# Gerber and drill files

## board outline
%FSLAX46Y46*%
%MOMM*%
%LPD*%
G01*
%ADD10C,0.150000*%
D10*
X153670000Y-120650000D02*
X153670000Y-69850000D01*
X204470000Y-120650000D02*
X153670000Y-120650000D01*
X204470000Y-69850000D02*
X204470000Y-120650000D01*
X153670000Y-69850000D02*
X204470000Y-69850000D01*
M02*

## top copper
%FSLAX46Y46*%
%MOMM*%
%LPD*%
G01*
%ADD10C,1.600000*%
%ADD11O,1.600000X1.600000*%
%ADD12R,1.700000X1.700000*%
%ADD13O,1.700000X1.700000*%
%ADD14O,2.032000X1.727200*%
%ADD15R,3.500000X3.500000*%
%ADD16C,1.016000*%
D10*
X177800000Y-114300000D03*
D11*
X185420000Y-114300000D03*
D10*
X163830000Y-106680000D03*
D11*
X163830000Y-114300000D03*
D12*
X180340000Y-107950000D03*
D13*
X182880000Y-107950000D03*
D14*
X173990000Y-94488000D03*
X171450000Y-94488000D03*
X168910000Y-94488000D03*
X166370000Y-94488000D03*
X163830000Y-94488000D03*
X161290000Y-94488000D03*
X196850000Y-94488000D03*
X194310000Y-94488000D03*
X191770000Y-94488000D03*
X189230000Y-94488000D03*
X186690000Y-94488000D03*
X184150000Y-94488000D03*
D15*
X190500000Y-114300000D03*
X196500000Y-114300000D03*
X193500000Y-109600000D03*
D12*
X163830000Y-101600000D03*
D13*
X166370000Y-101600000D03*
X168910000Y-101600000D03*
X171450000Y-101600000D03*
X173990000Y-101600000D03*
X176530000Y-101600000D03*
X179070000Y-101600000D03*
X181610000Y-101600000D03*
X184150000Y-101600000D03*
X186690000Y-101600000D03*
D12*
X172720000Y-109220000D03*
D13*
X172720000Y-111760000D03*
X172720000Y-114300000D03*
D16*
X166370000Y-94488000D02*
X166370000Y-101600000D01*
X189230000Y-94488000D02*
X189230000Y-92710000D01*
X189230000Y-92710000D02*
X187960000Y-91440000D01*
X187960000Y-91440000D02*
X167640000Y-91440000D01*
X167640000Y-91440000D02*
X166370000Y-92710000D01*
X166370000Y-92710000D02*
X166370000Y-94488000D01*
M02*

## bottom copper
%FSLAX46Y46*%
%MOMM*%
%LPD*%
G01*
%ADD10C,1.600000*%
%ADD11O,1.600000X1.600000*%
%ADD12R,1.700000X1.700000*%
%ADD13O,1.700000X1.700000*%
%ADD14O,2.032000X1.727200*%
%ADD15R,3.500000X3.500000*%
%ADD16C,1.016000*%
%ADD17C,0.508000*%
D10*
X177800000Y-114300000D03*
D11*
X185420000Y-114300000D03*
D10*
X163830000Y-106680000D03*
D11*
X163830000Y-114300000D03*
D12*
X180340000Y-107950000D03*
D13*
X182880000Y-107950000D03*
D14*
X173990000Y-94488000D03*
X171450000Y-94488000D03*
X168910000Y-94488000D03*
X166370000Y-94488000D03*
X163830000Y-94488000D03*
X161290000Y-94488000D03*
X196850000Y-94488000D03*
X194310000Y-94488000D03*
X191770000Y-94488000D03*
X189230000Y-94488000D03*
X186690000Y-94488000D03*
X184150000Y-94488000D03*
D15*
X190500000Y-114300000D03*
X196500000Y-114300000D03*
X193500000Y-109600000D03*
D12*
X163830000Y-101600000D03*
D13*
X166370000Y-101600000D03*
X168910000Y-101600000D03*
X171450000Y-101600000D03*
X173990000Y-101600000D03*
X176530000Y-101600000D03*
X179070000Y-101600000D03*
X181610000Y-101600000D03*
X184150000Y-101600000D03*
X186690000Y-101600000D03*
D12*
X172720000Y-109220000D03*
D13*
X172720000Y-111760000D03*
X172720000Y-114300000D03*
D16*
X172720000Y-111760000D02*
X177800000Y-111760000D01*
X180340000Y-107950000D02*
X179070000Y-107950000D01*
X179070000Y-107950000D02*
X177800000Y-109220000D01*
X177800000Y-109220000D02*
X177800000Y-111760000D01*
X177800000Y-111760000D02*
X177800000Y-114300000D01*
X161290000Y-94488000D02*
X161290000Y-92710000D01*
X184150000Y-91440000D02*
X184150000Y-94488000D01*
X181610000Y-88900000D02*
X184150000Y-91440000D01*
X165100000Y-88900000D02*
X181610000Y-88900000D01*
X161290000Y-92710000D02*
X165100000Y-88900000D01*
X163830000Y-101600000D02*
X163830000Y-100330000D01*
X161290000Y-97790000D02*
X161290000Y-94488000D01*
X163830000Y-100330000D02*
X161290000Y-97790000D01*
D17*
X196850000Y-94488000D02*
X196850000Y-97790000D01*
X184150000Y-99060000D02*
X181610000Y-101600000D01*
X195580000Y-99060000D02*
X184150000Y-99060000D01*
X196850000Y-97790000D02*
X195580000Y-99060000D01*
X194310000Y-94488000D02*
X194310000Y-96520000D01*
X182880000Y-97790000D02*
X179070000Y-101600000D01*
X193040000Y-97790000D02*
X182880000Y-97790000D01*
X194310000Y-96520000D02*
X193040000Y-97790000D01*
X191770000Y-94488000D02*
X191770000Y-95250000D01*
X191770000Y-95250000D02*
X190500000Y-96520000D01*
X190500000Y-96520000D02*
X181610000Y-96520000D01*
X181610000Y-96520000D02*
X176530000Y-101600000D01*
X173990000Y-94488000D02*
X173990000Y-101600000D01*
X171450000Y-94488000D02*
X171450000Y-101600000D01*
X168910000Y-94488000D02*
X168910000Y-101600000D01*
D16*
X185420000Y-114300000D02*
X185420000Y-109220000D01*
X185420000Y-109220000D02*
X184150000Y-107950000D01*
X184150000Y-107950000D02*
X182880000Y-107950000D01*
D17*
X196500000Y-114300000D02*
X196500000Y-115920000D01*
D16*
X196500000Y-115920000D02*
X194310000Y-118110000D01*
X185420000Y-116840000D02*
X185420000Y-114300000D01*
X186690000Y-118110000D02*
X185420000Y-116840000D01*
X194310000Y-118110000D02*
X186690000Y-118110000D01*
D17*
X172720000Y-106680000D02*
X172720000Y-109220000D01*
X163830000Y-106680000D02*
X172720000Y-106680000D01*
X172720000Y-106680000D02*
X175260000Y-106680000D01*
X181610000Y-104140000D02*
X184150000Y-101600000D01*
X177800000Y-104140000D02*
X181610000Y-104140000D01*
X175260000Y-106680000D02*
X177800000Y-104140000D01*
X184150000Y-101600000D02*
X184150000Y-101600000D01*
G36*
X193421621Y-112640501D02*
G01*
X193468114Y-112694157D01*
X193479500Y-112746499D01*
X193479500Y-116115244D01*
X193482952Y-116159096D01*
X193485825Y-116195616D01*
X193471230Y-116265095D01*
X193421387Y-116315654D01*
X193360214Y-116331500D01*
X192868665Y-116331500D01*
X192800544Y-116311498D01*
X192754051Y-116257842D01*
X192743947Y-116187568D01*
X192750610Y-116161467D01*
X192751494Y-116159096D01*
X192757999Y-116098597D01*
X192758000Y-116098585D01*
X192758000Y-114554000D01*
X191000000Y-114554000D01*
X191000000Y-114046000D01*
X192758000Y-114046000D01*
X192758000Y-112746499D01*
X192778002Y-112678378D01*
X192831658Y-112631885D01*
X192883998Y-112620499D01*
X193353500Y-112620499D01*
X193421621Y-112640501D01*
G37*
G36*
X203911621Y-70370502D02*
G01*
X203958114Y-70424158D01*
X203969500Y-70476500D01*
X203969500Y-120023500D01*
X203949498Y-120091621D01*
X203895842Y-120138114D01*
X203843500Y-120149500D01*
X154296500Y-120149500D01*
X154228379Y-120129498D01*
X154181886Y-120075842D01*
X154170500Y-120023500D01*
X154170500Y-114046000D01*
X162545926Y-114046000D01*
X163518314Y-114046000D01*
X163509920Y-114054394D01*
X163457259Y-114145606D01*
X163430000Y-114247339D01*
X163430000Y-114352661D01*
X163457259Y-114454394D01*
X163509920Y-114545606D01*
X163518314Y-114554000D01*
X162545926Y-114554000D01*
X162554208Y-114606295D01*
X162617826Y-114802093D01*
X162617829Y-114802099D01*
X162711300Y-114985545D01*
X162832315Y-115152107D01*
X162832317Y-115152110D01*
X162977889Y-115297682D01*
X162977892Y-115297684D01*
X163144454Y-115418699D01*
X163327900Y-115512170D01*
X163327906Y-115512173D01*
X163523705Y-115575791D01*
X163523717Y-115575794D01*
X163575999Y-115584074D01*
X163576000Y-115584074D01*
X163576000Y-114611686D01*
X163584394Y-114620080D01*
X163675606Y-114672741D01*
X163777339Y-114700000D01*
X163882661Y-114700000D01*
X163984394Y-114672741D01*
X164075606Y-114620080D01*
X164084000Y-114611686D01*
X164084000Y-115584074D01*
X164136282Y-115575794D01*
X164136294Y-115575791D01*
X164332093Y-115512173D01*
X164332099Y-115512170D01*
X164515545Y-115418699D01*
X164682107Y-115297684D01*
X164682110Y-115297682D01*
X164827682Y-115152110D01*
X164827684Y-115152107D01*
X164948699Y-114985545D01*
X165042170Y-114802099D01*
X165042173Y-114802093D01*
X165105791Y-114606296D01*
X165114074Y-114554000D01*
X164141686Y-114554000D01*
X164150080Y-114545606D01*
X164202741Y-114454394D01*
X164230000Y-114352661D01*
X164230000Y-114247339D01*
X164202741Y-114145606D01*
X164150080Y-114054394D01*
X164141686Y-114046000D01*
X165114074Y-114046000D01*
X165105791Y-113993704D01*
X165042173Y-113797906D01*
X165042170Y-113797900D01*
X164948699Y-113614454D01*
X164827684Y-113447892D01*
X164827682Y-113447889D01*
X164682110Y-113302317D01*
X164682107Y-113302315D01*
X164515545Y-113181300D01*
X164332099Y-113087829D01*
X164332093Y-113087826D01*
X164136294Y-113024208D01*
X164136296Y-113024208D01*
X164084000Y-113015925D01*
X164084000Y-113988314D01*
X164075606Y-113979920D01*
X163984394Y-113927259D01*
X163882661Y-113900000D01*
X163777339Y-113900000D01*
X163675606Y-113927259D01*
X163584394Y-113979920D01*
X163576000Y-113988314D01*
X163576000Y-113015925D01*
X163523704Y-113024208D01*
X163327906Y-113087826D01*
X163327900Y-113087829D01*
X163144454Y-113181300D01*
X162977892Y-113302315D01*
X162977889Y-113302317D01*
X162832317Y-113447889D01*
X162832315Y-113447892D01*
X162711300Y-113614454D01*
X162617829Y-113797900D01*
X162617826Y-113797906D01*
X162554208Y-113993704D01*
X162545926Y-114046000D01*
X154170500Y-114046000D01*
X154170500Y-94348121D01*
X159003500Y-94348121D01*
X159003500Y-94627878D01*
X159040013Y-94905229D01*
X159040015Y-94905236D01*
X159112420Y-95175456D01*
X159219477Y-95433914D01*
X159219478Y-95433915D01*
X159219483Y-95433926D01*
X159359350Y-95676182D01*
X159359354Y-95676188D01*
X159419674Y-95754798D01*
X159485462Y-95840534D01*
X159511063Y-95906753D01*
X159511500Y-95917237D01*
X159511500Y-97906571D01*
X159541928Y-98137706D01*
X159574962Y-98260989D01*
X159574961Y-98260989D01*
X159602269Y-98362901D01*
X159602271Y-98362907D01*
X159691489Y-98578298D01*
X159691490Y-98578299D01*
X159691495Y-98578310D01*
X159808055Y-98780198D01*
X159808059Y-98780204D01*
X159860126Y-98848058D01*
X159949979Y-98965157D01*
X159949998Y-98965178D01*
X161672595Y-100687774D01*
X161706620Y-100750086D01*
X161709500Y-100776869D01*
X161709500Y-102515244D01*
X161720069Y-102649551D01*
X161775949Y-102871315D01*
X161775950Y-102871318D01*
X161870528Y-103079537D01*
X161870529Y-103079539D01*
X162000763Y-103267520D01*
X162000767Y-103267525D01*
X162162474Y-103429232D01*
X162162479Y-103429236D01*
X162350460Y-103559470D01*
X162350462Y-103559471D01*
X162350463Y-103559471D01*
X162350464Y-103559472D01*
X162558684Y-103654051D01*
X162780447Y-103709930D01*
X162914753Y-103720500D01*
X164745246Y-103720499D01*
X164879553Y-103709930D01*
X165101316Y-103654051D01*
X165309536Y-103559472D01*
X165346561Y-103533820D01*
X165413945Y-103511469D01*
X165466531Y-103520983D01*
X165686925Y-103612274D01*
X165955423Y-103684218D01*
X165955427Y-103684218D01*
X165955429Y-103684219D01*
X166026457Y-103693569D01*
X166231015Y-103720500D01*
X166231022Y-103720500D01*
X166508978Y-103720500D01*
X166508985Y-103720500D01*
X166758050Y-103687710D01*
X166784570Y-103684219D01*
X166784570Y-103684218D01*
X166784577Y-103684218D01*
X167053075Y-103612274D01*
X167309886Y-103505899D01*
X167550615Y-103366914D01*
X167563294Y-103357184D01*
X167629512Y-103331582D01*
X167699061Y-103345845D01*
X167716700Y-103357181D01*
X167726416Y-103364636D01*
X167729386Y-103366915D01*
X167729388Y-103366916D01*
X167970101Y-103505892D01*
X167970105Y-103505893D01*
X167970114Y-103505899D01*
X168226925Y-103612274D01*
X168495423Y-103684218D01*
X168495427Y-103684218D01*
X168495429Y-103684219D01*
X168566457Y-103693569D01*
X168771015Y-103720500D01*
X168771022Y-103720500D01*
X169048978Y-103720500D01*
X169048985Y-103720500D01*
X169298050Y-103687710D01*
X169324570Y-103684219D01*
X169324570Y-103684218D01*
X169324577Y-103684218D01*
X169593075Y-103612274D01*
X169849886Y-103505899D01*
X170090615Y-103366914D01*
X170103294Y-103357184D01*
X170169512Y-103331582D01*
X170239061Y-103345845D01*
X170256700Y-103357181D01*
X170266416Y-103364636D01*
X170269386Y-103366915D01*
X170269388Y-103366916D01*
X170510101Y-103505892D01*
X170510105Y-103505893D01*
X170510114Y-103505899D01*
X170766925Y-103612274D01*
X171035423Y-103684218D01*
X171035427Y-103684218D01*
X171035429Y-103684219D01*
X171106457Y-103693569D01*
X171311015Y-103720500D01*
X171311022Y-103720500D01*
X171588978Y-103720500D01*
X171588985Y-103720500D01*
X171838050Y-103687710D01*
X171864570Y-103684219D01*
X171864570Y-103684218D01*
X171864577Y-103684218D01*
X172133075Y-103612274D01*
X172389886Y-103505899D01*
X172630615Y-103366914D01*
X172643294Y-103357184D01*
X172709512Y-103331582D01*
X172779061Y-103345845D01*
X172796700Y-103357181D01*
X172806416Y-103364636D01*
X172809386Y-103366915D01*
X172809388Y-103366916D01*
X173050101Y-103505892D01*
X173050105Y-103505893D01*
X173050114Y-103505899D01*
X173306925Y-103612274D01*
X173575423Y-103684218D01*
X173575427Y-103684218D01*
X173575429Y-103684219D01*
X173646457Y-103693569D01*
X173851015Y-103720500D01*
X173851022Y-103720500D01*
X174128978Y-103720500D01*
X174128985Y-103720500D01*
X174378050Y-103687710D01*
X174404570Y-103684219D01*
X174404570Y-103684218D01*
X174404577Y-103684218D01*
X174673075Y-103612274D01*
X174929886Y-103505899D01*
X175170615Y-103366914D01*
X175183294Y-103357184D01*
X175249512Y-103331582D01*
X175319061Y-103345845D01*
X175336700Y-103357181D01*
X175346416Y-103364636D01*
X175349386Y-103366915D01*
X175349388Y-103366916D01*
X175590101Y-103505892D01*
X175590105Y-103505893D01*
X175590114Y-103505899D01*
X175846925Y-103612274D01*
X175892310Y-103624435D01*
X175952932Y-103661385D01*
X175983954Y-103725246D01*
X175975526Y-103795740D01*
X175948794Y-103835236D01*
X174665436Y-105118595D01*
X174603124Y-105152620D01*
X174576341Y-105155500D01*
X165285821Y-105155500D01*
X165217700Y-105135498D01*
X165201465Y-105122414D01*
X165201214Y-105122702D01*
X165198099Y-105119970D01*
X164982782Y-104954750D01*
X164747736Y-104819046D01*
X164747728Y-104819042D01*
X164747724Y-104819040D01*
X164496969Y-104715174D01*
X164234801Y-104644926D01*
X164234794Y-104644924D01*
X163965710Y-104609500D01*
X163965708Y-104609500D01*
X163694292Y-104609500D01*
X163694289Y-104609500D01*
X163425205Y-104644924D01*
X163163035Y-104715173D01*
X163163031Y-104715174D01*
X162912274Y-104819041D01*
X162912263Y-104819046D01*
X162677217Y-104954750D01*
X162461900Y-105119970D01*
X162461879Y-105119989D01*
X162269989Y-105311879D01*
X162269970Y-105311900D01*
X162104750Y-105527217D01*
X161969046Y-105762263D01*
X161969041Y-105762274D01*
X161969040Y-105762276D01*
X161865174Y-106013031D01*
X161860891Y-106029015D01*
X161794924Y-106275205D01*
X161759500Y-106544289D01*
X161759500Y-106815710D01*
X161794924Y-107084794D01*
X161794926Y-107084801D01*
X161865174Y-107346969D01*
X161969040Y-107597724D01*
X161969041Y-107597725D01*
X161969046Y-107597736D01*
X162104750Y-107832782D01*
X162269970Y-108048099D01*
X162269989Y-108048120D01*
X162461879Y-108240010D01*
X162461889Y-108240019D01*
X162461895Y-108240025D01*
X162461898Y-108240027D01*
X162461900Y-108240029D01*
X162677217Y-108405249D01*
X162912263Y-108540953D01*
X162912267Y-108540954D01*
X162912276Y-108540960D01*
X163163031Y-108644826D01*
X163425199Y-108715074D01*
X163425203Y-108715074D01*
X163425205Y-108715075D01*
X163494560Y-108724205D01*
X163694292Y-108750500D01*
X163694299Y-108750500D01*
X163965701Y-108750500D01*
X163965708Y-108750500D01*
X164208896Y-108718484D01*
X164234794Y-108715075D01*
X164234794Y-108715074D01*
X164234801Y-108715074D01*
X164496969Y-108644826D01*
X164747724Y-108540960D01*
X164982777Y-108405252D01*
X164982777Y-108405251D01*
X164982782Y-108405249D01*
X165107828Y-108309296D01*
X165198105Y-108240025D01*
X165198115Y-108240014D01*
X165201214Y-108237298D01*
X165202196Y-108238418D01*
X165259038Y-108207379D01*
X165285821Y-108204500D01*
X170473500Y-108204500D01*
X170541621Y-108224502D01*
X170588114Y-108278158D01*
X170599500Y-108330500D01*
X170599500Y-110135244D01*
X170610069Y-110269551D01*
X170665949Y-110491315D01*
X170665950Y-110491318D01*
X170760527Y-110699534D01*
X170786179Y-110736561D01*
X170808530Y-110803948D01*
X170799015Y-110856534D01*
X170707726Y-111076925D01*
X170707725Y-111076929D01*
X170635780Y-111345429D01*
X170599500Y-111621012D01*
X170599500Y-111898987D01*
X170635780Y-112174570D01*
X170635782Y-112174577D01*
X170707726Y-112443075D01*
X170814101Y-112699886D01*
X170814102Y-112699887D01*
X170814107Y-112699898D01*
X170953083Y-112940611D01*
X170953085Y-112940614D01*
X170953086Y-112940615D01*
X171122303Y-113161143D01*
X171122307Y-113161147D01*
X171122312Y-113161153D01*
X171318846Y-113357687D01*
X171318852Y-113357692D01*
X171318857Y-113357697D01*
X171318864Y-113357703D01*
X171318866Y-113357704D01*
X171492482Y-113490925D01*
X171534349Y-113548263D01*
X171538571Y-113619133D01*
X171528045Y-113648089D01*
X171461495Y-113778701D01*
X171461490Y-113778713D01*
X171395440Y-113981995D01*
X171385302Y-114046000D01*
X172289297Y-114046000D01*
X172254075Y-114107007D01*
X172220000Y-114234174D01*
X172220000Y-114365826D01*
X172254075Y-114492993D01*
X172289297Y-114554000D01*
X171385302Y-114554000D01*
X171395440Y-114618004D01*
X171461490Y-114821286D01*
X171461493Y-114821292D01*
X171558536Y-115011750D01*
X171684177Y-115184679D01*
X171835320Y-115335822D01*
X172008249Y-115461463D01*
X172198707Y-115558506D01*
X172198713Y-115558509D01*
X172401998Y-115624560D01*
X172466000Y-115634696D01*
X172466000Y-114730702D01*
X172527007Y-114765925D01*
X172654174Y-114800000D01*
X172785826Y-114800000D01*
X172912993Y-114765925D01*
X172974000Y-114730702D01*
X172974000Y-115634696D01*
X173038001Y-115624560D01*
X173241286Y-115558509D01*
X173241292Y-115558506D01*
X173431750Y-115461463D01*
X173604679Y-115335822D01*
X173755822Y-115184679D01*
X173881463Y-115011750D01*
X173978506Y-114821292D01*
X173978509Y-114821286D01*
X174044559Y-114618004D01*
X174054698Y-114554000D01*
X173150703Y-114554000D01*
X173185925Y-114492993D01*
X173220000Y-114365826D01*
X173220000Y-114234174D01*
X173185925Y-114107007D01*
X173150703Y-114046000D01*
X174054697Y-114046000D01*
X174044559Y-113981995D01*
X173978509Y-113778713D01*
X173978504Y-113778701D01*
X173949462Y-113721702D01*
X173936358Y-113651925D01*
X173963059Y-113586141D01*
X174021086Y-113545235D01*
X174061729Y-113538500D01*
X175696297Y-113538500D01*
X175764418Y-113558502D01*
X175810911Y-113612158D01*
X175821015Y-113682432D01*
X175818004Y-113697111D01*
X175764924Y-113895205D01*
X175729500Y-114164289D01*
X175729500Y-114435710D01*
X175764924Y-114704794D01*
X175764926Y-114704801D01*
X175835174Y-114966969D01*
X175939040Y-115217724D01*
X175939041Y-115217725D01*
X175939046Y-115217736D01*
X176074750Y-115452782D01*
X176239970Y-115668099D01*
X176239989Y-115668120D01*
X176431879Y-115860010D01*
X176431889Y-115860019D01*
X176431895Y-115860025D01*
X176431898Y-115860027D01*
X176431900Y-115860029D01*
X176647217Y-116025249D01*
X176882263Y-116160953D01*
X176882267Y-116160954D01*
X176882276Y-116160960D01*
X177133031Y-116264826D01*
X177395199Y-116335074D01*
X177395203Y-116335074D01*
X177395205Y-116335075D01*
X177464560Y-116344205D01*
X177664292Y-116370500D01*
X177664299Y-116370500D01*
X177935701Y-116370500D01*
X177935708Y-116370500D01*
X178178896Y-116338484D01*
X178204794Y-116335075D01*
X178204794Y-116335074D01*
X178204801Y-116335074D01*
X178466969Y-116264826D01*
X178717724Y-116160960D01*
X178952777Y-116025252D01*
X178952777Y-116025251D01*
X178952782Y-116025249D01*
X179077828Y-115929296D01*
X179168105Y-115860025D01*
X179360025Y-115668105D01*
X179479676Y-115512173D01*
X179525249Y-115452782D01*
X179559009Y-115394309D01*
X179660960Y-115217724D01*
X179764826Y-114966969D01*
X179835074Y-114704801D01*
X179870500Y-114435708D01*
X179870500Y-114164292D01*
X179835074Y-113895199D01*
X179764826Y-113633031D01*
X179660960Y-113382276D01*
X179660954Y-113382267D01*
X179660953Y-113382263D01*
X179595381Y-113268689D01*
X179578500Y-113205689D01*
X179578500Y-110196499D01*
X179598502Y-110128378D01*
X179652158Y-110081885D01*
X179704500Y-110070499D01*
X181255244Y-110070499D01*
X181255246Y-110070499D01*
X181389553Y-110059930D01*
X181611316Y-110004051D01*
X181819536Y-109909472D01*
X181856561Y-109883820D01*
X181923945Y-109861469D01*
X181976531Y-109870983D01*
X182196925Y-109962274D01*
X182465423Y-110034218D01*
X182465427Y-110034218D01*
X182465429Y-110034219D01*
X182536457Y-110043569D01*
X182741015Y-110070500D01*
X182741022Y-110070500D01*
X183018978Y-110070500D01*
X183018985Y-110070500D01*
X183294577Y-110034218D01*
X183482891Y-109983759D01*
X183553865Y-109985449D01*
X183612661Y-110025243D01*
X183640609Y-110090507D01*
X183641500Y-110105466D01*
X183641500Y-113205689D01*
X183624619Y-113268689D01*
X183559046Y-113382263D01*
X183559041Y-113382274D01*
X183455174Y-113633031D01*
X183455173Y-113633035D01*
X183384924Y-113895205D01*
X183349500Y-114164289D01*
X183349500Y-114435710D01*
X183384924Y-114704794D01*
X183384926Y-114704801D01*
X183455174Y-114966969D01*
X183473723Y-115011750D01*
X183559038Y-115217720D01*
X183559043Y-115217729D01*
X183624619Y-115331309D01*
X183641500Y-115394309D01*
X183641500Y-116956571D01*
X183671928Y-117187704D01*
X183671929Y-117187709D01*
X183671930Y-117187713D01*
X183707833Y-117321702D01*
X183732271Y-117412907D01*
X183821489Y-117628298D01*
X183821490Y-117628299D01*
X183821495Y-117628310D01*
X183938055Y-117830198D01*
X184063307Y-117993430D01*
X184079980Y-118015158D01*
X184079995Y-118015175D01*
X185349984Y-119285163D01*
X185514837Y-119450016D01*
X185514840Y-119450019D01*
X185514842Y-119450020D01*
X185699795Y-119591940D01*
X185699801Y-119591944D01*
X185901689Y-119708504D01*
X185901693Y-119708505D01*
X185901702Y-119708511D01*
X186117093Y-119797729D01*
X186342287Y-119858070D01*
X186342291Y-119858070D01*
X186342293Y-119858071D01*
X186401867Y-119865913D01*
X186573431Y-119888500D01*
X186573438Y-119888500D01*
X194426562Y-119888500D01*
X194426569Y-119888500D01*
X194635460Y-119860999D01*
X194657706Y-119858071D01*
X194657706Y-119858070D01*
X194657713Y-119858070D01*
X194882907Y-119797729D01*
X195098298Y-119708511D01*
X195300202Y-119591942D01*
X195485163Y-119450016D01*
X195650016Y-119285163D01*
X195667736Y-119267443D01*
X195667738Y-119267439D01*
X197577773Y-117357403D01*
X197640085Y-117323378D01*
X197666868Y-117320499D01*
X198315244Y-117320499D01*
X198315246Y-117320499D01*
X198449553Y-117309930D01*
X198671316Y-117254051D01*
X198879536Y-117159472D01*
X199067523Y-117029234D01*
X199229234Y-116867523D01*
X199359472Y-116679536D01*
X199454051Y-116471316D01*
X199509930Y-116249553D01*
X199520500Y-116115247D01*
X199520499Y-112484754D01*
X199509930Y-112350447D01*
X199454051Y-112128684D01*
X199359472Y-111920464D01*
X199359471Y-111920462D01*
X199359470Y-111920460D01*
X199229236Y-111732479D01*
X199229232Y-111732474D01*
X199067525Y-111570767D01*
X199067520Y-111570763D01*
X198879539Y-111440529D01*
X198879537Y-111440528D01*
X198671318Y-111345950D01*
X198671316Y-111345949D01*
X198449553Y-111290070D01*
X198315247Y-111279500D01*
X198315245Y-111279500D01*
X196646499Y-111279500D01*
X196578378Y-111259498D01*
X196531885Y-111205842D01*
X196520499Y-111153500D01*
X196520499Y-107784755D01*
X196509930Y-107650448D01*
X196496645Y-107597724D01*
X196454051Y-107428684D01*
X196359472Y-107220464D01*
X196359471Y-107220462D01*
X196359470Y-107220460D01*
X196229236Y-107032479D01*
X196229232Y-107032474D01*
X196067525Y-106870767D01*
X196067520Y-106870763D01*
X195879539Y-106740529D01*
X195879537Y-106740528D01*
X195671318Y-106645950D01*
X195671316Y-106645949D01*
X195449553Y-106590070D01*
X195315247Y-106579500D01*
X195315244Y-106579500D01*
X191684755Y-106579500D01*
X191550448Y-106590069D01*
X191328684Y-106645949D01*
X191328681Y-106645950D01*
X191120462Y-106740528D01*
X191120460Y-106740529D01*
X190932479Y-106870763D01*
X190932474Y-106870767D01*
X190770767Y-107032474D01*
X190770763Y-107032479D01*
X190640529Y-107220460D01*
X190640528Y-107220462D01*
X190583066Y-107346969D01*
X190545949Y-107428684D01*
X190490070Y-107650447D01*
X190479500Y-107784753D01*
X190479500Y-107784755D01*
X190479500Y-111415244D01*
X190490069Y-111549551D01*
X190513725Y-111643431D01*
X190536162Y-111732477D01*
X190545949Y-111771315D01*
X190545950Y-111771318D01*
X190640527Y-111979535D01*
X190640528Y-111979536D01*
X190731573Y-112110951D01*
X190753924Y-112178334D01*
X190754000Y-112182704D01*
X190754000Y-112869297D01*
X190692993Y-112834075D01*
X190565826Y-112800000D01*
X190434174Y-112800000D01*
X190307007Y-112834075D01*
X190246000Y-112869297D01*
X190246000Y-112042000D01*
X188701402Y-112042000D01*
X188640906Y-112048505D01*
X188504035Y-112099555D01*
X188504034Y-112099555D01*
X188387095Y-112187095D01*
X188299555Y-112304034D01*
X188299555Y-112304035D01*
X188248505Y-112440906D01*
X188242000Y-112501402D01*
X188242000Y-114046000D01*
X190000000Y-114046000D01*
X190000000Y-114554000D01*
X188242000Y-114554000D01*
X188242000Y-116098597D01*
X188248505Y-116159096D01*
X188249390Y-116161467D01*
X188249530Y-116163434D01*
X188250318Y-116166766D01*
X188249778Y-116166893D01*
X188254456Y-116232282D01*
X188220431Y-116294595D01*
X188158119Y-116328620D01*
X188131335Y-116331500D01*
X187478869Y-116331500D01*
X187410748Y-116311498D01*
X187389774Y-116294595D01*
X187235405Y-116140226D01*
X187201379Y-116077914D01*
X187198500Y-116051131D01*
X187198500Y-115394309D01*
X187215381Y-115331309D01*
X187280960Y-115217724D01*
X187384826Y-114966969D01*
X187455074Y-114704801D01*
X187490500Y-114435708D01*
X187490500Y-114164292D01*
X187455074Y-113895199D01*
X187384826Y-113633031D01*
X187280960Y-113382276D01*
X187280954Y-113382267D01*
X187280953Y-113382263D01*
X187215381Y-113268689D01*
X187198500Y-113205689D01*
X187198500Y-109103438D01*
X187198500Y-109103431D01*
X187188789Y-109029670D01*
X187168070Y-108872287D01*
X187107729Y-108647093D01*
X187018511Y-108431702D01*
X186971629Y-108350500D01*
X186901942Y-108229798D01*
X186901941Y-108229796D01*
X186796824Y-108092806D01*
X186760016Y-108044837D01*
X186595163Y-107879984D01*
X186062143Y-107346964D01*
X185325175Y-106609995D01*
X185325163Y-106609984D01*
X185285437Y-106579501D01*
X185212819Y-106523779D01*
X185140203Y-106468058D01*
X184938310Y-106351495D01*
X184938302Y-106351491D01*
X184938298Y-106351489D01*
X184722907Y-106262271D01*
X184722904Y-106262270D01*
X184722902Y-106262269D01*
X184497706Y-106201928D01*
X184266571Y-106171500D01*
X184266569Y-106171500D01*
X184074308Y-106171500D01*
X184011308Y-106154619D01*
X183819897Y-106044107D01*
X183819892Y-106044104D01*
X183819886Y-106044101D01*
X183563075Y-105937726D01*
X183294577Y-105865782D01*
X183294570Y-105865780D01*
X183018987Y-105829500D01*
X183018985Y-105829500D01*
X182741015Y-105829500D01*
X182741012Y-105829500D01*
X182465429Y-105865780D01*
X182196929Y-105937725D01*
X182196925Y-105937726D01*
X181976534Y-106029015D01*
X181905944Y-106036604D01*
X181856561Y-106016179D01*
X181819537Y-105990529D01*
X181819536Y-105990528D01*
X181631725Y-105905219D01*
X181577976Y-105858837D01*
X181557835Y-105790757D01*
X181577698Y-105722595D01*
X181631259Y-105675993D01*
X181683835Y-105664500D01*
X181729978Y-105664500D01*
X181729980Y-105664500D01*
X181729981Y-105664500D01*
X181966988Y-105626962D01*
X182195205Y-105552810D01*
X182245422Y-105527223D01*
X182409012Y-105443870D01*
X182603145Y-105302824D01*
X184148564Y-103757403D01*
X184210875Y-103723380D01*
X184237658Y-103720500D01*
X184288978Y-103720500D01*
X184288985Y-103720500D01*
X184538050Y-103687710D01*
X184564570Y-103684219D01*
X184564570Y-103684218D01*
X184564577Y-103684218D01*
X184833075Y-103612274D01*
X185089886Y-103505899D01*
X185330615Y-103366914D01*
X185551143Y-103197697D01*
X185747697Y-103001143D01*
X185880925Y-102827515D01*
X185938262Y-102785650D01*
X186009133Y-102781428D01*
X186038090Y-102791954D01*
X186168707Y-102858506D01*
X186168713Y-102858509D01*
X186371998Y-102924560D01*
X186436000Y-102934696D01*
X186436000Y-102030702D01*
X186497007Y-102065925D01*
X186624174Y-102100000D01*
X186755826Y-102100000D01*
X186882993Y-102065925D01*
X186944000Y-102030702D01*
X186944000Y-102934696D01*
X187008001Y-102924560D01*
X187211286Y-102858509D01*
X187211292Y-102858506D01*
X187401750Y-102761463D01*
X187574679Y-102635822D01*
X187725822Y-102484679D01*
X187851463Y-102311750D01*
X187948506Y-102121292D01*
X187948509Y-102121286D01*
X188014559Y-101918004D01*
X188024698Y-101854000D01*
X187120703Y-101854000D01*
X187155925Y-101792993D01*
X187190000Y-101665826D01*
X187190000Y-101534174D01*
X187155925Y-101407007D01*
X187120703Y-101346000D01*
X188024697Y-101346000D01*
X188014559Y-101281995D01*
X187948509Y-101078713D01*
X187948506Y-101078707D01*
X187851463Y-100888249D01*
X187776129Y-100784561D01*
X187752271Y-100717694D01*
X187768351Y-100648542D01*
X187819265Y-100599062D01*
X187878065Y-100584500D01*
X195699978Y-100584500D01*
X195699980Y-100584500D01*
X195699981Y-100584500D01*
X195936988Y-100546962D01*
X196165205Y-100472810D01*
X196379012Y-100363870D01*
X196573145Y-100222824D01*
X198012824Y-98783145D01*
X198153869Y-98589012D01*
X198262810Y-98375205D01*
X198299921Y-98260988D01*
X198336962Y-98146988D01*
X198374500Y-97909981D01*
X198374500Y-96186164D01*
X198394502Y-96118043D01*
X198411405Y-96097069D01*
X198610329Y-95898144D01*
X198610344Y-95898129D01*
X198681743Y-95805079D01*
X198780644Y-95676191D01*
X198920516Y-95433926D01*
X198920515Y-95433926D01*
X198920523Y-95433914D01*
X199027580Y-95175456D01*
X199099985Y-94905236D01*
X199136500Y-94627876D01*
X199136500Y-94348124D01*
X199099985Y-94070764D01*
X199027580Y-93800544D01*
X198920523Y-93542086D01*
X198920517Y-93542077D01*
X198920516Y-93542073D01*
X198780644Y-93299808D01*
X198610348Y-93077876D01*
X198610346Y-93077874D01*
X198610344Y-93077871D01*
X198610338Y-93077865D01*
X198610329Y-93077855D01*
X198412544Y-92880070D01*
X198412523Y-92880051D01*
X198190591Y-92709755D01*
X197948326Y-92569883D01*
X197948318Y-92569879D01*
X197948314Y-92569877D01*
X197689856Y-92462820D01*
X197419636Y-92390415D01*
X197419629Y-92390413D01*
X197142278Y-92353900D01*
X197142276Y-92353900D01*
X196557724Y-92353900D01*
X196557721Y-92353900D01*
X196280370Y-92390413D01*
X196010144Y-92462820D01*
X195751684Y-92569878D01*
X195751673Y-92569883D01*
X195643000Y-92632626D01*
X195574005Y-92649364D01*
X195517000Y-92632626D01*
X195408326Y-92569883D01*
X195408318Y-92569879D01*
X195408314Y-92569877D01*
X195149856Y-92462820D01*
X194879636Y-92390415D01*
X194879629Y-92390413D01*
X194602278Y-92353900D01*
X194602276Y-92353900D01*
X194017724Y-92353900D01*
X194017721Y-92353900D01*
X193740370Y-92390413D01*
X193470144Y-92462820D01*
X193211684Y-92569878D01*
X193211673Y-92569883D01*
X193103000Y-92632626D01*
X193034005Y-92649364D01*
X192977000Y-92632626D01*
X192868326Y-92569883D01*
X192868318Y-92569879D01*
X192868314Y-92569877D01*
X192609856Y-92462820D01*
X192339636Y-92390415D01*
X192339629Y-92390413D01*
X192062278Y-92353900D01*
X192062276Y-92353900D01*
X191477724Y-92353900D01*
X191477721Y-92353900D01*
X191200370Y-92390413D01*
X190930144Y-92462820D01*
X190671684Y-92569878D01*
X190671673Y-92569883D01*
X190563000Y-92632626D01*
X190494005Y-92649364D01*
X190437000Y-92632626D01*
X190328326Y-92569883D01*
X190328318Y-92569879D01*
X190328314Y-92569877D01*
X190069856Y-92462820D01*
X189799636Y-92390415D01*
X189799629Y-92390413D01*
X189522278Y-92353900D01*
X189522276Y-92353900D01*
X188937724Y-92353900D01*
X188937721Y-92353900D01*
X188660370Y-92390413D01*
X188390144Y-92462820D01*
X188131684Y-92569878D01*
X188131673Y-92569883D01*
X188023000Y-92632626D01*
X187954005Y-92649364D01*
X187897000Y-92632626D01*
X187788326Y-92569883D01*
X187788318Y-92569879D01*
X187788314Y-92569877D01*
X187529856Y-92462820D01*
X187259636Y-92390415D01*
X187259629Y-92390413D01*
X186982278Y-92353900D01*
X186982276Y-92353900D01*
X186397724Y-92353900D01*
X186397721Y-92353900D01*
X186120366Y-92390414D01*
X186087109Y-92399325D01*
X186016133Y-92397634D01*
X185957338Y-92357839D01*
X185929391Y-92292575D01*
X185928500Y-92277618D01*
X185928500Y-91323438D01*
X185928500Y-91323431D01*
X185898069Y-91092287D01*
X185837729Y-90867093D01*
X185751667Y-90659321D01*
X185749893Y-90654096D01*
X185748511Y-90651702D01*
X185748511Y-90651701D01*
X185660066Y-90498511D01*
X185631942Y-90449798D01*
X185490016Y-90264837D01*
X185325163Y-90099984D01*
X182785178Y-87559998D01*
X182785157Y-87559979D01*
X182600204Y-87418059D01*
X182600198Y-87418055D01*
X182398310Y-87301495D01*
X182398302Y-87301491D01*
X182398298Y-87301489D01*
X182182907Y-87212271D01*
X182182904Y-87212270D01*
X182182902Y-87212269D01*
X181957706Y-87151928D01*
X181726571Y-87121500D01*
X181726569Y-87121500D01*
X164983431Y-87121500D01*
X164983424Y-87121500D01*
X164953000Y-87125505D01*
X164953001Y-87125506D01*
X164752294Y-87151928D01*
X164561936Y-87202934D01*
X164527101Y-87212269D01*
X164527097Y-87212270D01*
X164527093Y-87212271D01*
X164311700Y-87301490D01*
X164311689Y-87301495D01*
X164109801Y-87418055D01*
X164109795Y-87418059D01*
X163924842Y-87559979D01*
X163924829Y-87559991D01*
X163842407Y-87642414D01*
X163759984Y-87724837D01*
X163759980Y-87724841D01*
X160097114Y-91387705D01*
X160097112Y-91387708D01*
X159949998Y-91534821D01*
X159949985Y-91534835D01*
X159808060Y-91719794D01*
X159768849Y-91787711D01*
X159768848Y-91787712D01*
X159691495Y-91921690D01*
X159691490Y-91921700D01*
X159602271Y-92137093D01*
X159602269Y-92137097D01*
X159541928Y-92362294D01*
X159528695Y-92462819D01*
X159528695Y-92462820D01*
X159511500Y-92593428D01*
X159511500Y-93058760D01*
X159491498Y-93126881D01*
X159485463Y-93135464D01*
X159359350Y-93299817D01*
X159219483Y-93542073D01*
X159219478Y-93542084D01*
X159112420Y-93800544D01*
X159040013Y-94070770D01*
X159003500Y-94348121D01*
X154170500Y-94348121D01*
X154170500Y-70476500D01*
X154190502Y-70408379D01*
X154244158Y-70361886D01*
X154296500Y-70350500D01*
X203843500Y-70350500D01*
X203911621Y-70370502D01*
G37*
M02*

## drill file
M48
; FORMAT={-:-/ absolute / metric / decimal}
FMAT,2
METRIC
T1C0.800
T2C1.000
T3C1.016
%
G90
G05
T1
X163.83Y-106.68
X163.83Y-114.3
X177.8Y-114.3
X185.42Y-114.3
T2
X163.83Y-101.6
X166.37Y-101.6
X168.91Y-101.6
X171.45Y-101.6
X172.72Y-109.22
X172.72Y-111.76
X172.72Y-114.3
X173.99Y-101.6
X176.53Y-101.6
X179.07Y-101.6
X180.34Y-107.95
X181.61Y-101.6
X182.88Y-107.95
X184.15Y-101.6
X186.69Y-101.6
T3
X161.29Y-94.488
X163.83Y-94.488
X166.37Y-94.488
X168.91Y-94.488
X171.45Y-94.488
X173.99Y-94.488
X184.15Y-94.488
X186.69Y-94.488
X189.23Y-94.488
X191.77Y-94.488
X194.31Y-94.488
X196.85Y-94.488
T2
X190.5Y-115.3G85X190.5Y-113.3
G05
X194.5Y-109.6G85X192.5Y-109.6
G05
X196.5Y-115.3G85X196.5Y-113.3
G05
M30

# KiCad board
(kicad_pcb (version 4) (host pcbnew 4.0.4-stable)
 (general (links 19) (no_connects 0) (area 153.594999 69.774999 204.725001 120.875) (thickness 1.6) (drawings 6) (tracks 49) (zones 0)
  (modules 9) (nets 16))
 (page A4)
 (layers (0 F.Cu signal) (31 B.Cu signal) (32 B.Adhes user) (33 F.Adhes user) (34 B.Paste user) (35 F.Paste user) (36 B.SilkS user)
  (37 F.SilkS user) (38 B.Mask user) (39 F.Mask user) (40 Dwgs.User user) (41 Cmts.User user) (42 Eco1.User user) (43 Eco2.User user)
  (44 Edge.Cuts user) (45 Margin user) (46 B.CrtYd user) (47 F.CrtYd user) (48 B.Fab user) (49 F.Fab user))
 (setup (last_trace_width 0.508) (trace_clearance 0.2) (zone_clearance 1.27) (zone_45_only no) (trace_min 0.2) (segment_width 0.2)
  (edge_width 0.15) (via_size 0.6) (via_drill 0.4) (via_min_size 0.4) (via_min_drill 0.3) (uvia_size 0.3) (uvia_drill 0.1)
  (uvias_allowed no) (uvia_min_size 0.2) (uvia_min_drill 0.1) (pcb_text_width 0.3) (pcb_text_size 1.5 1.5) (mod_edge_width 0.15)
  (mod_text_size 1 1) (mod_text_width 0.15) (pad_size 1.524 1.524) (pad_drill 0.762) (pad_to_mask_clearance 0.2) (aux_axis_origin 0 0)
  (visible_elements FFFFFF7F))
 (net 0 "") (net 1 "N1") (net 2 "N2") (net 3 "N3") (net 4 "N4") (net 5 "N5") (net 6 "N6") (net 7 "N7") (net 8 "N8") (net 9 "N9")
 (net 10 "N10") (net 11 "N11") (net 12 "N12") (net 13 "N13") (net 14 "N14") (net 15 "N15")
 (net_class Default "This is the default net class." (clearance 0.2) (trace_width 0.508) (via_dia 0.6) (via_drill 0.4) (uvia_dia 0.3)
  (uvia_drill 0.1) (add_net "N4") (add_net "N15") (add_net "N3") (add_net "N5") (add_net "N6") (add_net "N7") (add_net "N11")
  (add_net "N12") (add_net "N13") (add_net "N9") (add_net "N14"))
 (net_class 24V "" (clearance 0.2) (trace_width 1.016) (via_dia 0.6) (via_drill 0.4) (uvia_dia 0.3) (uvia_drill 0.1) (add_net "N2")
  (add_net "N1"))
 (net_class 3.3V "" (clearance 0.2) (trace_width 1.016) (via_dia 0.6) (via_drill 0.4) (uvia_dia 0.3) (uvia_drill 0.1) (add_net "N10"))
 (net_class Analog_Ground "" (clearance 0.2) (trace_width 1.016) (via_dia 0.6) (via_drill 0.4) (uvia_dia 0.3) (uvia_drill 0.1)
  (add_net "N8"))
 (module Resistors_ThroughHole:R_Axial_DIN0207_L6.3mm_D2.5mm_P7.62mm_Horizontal (layer F.Cu) (at 177.8 114.3)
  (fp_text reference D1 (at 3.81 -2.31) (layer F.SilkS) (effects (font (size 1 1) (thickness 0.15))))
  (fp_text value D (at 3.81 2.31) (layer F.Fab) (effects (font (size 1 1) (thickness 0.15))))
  (pad 1 thru_hole circle (at 0 0) (size 1.6 1.6) (drill 0.8) (layers *.Cu *.Mask) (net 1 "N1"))
  (pad 2 thru_hole oval (at 7.62 0) (size 1.6 1.6) (drill 0.8) (layers *.Cu *.Mask) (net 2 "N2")))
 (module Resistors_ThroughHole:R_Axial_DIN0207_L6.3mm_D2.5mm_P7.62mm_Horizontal (layer F.Cu) (at 163.83 106.68 270)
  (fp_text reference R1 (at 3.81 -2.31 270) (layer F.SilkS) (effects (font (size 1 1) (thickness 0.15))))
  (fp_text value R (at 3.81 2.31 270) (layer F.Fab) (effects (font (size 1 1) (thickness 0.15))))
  (pad 1 thru_hole circle (at 0 0 270) (size 1.6 1.6) (drill 0.8) (layers *.Cu *.Mask) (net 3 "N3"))
  (pad 2 thru_hole oval (at 7.62 0 270) (size 1.6 1.6) (drill 0.8) (layers *.Cu *.Mask) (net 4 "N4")))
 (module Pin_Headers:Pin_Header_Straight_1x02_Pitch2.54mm (layer F.Cu) (at 180.34 107.95 90)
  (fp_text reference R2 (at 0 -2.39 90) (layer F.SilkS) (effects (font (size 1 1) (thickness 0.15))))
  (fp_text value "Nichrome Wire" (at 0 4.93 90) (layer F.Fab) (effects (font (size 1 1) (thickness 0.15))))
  (pad 1 thru_hole rect (at 0 0 90) (size 1.7 1.7) (drill 1) (layers *.Cu *.Mask) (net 1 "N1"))
  (pad 2 thru_hole oval (at 0 2.54 90) (size 1.7 1.7) (drill 1) (layers *.Cu *.Mask) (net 2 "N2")))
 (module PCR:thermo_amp (layer F.Cu) (at 167.64 85.09)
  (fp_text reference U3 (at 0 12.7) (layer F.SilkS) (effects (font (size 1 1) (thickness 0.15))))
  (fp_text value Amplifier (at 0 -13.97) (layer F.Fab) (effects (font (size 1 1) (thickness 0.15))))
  (pad 6 thru_hole oval (at 6.35 9.398) (size 2.032 1.7272) (drill 1.016) (layers *.Cu *.Mask) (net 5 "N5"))
  (pad 5 thru_hole oval (at 3.81 9.398) (size 2.032 1.7272) (drill 1.016) (layers *.Cu *.Mask) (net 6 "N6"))
  (pad 4 thru_hole oval (at 1.27 9.398) (size 2.032 1.7272) (drill 1.016) (layers *.Cu *.Mask) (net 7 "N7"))
  (pad 3 thru_hole oval (at -1.27 9.398) (size 2.032 1.7272) (drill 1.016) (layers *.Cu *.Mask) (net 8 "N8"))
  (pad 2 thru_hole oval (at -3.81 9.398) (size 2.032 1.7272) (drill 1.016) (layers *.Cu *.Mask) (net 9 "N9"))
  (pad 1 thru_hole oval (at -6.35 9.398) (size 2.032 1.7272) (drill 1.016) (layers *.Cu *.Mask) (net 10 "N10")))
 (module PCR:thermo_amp (layer F.Cu) (at 190.5 85.09)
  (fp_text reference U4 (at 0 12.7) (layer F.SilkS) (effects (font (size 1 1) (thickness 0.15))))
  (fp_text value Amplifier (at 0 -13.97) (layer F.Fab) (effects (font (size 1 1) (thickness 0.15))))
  (pad 6 thru_hole oval (at 6.35 9.398) (size 2.032 1.7272) (drill 1.016) (layers *.Cu *.Mask) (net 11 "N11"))
  (pad 5 thru_hole oval (at 3.81 9.398) (size 2.032 1.7272) (drill 1.016) (layers *.Cu *.Mask) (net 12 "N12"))
  (pad 4 thru_hole oval (at 1.27 9.398) (size 2.032 1.7272) (drill 1.016) (layers *.Cu *.Mask) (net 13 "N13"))
  (pad 3 thru_hole oval (at -1.27 9.398) (size 2.032 1.7272) (drill 1.016) (layers *.Cu *.Mask) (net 8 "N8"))
  (pad 2 thru_hole oval (at -3.81 9.398) (size 2.032 1.7272) (drill 1.016) (layers *.Cu *.Mask) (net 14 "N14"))
  (pad 1 thru_hole oval (at -6.35 9.398) (size 2.032 1.7272) (drill 1.016) (layers *.Cu *.Mask) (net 10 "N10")))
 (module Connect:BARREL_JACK (layer F.Cu) (at 190.5 114.3 180)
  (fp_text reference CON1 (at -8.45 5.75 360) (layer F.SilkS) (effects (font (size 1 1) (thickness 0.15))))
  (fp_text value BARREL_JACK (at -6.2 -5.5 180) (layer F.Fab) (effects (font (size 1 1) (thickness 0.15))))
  (pad 1 thru_hole rect (at 0 0 180) (size 3.5 3.5) (drill oval 1 3) (layers *.Cu *.Mask) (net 4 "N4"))
  (pad 2 thru_hole rect (at -6 0 180) (size 3.5 3.5) (drill oval 1 3) (layers *.Cu *.Mask) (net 2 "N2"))
  (pad 3 thru_hole rect (at -3 4.7 180) (size 3.5 3.5) (drill oval 3 1) (layers *.Cu *.Mask) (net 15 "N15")))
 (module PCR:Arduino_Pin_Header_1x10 (layer F.Cu) (at 163.83 101.6 90)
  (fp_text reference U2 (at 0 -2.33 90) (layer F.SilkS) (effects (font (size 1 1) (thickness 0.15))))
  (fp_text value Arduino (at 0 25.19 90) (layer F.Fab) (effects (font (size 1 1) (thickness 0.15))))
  (pad 13 thru_hole rect (at 0 0 90) (size 1.7 1.7) (drill 1) (layers *.Cu *.Mask) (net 10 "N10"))
  (pad 17 thru_hole oval (at 0 2.54 90) (size 1.7 1.7) (drill 1) (layers *.Cu *.Mask) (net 8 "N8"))
  (pad 12 thru_hole oval (at 0 5.08 90) (size 1.7 1.7) (drill 1) (layers *.Cu *.Mask) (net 7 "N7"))
  (pad 11 thru_hole oval (at 0 7.62 90) (size 1.7 1.7) (drill 1) (layers *.Cu *.Mask) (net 6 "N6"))
  (pad 10 thru_hole oval (at 0 10.16 90) (size 1.7 1.7) (drill 1) (layers *.Cu *.Mask) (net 5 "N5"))
  (pad 6 thru_hole oval (at 0 12.7 90) (size 1.7 1.7) (drill 1) (layers *.Cu *.Mask) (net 13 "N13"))
  (pad 5 thru_hole oval (at 0 15.24 90) (size 1.7 1.7) (drill 1) (layers *.Cu *.Mask) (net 12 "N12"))
  (pad 4 thru_hole oval (at 0 17.78 90) (size 1.7 1.7) (drill 1) (layers *.Cu *.Mask) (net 11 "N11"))
  (pad 3 thru_hole oval (at 0 20.32 90) (size 1.7 1.7) (drill 1) (layers *.Cu *.Mask) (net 3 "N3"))
  (pad 16 thru_hole oval (at 0 22.86 90) (size 1.7 1.7) (drill 1) (layers *.Cu *.Mask) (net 4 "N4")))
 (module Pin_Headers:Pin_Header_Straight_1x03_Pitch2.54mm (layer F.Cu) (at 172.72 109.22)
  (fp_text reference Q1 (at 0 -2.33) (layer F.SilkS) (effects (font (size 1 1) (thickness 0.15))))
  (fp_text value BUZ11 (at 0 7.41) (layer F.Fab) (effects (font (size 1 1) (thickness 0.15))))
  (pad 1 thru_hole rect (at 0 0) (size 1.7 1.7) (drill 1) (layers *.Cu *.Mask) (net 3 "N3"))
  (pad 2 thru_hole oval (at 0 2.54) (size 1.7 1.7) (drill 1) (layers *.Cu *.Mask) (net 1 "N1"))
  (pad 3 thru_hole oval (at 0 5.08) (size 1.7 1.7) (drill 1) (layers *.Cu *.Mask) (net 4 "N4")))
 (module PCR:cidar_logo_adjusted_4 (layer B.Cu) (at 179.705 78.74 180)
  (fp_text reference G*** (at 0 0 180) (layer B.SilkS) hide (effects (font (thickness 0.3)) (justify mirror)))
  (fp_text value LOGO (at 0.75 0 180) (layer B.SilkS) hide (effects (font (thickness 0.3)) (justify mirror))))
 (gr_line (start 153.67 120.65) (end 153.67 69.85) (angle 90) (layer Edge.Cuts) (width 0.15))
 (gr_line (start 204.47 120.65) (end 153.67 120.65) (angle 90) (layer Edge.Cuts) (width 0.15))
 (gr_line (start 204.47 69.85) (end 204.47 120.65) (angle 90) (layer Edge.Cuts) (width 0.15))
 (gr_line (start 153.67 69.85) (end 204.47 69.85) (angle 90) (layer Edge.Cuts) (width 0.15))
 (segment (start 172.72 111.76) (end 177.8 111.76) (width 1.016) (layer B.Cu) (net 1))
 (segment (start 180.34 107.95) (end 179.07 107.95) (width 1.016) (layer B.Cu) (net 1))
 (segment (start 179.07 107.95) (end 177.8 109.22) (width 1.016) (layer B.Cu) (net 1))
 (segment (start 177.8 109.22) (end 177.8 111.76) (width 1.016) (layer B.Cu) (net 1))
 (segment (start 177.8 111.76) (end 177.8 114.3) (width 1.016) (layer B.Cu) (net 1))
 (segment (start 161.29 94.488) (end 161.29 92.71) (width 1.016) (layer B.Cu) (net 10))
 (segment (start 184.15 91.44) (end 184.15 94.488) (width 1.016) (layer B.Cu) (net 10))
 (segment (start 181.61 88.9) (end 184.15 91.44) (width 1.016) (layer B.Cu) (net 10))
 (segment (start 165.1 88.9) (end 181.61 88.9) (width 1.016) (layer B.Cu) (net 10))
 (segment (start 161.29 92.71) (end 165.1 88.9) (width 1.016) (layer B.Cu) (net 10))
 (segment (start 163.83 101.6) (end 163.83 100.33) (width 1.016) (layer B.Cu) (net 10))
 (segment (start 161.29 97.79) (end 161.29 94.488) (width 1.016) (layer B.Cu) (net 10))
 (segment (start 163.83 100.33) (end 161.29 97.79) (width 1.016) (layer B.Cu) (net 10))
 (segment (start 196.85 94.488) (end 196.85 97.79) (width 0.508) (layer B.Cu) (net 11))
 (segment (start 184.15 99.06) (end 181.61 101.6) (width 0.508) (layer B.Cu) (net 11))
 (segment (start 195.58 99.06) (end 184.15 99.06) (width 0.508) (layer B.Cu) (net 11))
 (segment (start 196.85 97.79) (end 195.58 99.06) (width 0.508) (layer B.Cu) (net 11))
 (segment (start 194.31 94.488) (end 194.31 96.52) (width 0.508) (layer B.Cu) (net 12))
 (segment (start 182.88 97.79) (end 179.07 101.6) (width 0.508) (layer B.Cu) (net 12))
 (segment (start 193.04 97.79) (end 182.88 97.79) (width 0.508) (layer B.Cu) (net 12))
 (segment (start 194.31 96.52) (end 193.04 97.79) (width 0.508) (layer B.Cu) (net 12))
 (segment (start 191.77 94.488) (end 191.77 95.25) (width 0.508) (layer B.Cu) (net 13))
 (segment (start 191.77 95.25) (end 190.5 96.52) (width 0.508) (layer B.Cu) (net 13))
 (segment (start 190.5 96.52) (end 181.61 96.52) (width 0.508) (layer B.Cu) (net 13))
 (segment (start 181.61 96.52) (end 176.53 101.6) (width 0.508) (layer B.Cu) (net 13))
 (segment (start 173.99 94.488) (end 173.99 101.6) (width 0.508) (layer B.Cu) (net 5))
 (segment (start 171.45 94.488) (end 171.45 101.6) (width 0.508) (layer B.Cu) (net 6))
 (segment (start 168.91 94.488) (end 168.91 101.6) (width 0.508) (layer B.Cu) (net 7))
 (segment (start 166.37 94.488) (end 166.37 101.6) (width 1.016) (layer F.Cu) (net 8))
 (segment (start 189.23 94.488) (end 189.23 92.71) (width 1.016) (layer F.Cu) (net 8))
 (segment (start 189.23 92.71) (end 187.96 91.44) (width 1.016) (layer F.Cu) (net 8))
 (segment (start 187.96 91.44) (end 167.64 91.44) (width 1.016) (layer F.Cu) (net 8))
 (segment (start 167.64 91.44) (end 166.37 92.71) (width 1.016) (layer F.Cu) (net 8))
 (segment (start 166.37 92.71) (end 166.37 94.488) (width 1.016) (layer F.Cu) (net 8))
 (segment (start 185.42 114.3) (end 185.42 109.22) (width 1.016) (layer B.Cu) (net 2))
 (segment (start 185.42 109.22) (end 184.15 107.95) (width 1.016) (layer B.Cu) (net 2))
 (segment (start 184.15 107.95) (end 182.88 107.95) (width 1.016) (layer B.Cu) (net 2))
 (segment (start 196.5 114.3) (end 196.5 115.92) (width 0.508) (layer B.Cu) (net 2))
 (segment (start 196.5 115.92) (end 194.31 118.11) (width 1.016) (layer B.Cu) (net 2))
 (segment (start 185.42 116.84) (end 185.42 114.3) (width 1.016) (layer B.Cu) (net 2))
 (segment (start 186.69 118.11) (end 185.42 116.84) (width 1.016) (layer B.Cu) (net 2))
 (segment (start 194.31 118.11) (end 186.69 118.11) (width 1.016) (layer B.Cu) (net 2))
 (segment (start 172.72 106.68) (end 172.72 109.22) (width 0.508) (layer B.Cu) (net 3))
 (segment (start 163.83 106.68) (end 172.72 106.68) (width 0.508) (layer B.Cu) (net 3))
 (segment (start 172.72 106.68) (end 175.26 106.68) (width 0.508) (layer B.Cu) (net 3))
 (segment (start 181.61 104.14) (end 184.15 101.6) (width 0.508) (layer B.Cu) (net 3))
 (segment (start 177.8 104.14) (end 181.61 104.14) (width 0.508) (layer B.Cu) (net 3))
 (segment (start 175.26 106.68) (end 177.8 104.14) (width 0.508) (layer B.Cu) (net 3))
 (segment (start 184.15 101.6) (end 184.15 101.6) (width 0.508) (layer B.Cu) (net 3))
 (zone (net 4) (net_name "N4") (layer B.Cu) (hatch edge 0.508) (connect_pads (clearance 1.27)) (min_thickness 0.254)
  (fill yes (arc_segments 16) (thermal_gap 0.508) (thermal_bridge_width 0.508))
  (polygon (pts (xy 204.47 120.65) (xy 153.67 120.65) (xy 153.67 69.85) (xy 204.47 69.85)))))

